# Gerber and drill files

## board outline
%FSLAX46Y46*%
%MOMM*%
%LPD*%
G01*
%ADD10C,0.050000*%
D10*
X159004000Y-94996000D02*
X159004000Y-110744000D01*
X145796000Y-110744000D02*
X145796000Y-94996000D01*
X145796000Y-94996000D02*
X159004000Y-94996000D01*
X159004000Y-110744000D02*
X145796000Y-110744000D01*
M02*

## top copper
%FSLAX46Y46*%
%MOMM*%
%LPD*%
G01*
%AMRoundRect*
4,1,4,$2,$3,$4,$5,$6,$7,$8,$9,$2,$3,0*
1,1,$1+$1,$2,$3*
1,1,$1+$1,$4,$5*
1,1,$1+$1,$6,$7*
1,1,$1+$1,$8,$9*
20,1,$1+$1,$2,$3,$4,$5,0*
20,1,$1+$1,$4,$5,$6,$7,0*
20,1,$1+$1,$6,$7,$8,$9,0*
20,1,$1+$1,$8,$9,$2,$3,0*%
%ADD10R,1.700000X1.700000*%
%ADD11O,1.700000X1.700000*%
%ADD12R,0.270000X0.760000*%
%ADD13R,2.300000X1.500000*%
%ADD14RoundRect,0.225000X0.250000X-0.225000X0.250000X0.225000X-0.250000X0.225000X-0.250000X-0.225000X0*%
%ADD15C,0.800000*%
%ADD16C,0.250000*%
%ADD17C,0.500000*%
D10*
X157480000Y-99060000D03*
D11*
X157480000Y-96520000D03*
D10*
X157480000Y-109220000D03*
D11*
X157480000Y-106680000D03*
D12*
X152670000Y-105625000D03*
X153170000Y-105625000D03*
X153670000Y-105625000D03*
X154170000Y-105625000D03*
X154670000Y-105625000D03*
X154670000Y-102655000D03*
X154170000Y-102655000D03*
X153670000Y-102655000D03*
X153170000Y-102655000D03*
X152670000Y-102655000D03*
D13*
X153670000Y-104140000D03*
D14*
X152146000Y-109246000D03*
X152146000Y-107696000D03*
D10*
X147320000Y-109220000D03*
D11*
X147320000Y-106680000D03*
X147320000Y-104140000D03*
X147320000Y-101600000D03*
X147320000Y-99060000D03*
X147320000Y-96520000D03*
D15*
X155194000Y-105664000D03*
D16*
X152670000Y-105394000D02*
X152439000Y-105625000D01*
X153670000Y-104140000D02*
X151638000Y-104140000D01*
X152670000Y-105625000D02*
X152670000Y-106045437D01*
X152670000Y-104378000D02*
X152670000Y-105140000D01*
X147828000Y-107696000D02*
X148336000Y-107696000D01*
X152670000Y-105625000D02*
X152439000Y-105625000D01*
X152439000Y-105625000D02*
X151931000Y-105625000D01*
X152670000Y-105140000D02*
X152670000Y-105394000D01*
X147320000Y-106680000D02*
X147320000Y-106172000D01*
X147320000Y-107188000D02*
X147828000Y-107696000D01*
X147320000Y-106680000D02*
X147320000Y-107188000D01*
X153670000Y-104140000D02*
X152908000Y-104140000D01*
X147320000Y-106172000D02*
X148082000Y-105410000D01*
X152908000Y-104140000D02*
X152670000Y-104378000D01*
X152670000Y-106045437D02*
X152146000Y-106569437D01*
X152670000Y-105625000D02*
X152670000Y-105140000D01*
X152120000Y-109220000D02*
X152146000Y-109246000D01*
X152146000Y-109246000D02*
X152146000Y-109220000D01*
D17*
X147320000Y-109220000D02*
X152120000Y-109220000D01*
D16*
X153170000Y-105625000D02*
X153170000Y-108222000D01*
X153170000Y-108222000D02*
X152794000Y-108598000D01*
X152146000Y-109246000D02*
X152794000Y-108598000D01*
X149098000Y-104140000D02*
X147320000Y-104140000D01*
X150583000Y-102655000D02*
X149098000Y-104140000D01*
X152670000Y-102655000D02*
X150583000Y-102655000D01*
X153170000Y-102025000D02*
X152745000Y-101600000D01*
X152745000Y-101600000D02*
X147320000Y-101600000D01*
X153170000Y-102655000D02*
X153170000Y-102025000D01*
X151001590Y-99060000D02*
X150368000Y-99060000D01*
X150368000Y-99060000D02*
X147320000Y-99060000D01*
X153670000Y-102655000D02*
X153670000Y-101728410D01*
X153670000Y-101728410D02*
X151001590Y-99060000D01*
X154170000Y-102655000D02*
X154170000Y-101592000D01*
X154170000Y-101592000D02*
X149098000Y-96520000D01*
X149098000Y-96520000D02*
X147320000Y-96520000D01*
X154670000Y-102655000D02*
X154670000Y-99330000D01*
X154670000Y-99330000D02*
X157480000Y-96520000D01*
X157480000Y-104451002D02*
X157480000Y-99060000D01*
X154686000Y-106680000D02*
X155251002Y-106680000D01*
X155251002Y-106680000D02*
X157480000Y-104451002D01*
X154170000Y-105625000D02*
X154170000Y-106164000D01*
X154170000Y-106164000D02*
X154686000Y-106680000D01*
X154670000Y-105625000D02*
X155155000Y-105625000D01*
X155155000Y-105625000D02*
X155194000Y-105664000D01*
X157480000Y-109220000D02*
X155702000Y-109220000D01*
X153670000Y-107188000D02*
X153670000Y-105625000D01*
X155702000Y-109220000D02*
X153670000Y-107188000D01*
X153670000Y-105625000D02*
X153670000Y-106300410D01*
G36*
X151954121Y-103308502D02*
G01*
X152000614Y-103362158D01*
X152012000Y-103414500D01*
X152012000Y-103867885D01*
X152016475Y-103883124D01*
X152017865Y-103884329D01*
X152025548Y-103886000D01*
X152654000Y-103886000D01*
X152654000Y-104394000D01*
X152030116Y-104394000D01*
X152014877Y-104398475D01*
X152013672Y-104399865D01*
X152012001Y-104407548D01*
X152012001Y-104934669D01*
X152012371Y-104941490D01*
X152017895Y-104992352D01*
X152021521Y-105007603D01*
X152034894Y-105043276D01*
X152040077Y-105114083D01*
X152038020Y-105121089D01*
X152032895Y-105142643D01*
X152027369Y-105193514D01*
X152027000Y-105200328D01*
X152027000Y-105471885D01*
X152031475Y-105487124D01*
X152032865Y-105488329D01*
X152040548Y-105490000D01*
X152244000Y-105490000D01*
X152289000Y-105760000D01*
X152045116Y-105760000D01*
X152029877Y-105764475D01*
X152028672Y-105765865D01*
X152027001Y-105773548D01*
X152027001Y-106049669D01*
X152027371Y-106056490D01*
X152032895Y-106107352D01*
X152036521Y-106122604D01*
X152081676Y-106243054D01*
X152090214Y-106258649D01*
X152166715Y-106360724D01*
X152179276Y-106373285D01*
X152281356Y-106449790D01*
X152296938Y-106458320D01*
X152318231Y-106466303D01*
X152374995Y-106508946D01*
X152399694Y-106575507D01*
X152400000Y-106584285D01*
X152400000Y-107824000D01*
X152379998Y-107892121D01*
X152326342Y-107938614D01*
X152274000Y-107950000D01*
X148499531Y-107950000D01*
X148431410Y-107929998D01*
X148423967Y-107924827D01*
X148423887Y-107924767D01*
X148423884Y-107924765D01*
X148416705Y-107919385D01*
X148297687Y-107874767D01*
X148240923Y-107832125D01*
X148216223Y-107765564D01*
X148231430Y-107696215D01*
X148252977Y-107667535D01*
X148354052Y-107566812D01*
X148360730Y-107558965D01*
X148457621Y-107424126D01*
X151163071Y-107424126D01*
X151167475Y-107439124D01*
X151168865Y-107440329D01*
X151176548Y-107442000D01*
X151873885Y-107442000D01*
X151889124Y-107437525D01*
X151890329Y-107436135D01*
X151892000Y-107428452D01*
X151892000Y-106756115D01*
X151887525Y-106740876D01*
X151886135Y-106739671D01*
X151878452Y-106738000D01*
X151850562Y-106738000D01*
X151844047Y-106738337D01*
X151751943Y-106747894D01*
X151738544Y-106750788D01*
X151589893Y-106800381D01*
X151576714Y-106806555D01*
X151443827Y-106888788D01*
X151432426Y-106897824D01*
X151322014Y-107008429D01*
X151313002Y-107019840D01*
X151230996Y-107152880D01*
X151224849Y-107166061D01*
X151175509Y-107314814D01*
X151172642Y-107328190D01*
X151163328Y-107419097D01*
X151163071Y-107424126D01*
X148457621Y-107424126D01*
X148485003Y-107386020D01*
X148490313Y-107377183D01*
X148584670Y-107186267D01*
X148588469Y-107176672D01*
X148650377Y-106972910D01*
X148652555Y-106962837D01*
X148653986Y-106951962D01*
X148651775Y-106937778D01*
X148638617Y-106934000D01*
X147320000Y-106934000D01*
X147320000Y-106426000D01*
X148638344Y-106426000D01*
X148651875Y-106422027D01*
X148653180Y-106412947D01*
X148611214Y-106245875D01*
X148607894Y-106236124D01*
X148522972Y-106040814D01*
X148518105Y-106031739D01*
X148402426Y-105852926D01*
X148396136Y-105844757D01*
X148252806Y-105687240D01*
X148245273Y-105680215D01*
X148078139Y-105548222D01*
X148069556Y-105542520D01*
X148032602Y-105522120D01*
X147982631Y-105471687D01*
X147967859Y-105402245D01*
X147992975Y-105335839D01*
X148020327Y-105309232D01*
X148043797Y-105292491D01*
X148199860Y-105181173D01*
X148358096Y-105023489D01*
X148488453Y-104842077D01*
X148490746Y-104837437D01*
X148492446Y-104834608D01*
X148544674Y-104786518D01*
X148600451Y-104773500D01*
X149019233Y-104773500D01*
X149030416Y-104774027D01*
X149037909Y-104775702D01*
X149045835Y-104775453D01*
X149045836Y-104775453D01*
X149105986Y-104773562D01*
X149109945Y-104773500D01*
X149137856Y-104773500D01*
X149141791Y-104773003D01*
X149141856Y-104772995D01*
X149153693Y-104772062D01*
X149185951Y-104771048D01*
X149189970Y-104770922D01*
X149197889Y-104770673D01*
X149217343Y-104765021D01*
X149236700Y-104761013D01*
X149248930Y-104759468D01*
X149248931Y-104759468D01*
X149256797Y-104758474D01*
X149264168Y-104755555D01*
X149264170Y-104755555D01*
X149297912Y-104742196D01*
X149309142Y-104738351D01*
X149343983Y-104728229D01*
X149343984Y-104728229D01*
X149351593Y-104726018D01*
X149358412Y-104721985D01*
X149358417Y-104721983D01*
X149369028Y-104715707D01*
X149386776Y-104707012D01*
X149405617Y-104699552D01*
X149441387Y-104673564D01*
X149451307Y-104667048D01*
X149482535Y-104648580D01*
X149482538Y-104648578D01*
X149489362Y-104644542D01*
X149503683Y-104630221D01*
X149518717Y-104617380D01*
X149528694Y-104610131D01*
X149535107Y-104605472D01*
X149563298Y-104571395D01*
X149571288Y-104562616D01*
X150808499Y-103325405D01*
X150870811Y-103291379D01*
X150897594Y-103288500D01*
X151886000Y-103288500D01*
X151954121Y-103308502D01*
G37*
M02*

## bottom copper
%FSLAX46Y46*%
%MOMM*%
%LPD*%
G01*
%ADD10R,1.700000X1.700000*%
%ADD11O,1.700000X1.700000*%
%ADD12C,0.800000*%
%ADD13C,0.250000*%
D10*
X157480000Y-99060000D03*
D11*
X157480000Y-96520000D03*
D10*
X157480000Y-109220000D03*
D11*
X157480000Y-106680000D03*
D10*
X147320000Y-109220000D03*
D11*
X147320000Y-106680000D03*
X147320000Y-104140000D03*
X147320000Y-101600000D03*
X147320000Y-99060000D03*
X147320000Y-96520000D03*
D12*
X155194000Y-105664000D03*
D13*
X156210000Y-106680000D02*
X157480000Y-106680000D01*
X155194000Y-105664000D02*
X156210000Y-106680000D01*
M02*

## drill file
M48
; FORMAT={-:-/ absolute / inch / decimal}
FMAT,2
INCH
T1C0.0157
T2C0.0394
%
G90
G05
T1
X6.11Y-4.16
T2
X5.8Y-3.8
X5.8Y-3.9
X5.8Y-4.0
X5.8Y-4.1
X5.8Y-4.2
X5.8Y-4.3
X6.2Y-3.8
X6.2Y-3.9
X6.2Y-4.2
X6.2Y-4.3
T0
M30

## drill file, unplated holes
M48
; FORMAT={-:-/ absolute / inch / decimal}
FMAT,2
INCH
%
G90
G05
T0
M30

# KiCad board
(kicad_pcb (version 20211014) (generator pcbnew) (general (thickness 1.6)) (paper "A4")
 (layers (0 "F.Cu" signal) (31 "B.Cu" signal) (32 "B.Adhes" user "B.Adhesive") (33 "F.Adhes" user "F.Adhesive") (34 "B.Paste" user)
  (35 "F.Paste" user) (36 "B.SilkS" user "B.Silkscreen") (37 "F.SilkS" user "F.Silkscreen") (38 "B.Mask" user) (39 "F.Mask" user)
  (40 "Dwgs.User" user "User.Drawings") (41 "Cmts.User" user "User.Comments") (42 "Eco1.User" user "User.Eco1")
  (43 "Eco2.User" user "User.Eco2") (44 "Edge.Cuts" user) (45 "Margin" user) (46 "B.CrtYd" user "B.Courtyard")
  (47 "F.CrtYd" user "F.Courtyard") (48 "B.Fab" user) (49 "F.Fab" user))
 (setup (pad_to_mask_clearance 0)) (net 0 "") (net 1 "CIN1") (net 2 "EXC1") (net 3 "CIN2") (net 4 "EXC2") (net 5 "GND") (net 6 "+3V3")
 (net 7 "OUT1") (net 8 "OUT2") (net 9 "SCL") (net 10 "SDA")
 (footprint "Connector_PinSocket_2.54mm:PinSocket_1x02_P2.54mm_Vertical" (layer "F.Cu") (at 157.48 99.06 180)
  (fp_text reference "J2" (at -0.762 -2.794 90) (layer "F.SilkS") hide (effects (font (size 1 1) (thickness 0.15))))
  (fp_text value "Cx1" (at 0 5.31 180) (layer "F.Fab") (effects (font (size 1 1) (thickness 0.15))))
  (pad "1" thru_hole rect locked (at 0 0 180) (size 1.7 1.7) (drill 1) (layers *.Cu *.Mask) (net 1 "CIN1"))
  (pad "2" thru_hole oval locked (at 0 2.54 180) (size 1.7 1.7) (drill 1) (layers *.Cu *.Mask) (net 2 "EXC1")))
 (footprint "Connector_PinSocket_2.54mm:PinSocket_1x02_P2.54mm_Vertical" (layer "F.Cu") (at 157.48 109.22 180)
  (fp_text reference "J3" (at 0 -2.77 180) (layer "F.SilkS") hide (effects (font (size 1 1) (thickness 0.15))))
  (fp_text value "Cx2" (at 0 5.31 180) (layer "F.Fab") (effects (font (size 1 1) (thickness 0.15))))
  (pad "1" thru_hole rect locked (at 0 0 180) (size 1.7 1.7) (drill 1) (layers *.Cu *.Mask) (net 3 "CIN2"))
  (pad "2" thru_hole oval locked (at 0 2.54 180) (size 1.7 1.7) (drill 1) (layers *.Cu *.Mask) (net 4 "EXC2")))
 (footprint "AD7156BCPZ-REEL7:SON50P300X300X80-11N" (layer "F.Cu") (at 153.67 104.14 90)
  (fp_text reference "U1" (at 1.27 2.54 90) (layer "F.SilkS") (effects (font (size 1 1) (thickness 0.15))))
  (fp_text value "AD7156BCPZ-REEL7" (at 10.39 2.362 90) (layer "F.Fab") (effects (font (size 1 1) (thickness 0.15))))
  (pad "1" smd rect locked (at -1.485 -1 90) (size 0.76 0.27) (layers "F.Cu" "F.Paste" "F.Mask") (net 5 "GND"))
  (pad "2" smd rect locked (at -1.485 -0.5 90) (size 0.76 0.27) (layers "F.Cu" "F.Paste" "F.Mask") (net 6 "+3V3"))
  (pad "3" smd rect locked (at -1.485 0 90) (size 0.76 0.27) (layers "F.Cu" "F.Paste" "F.Mask") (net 3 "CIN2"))
  (pad "4" smd rect locked (at -1.485 0.5 90) (size 0.76 0.27) (layers "F.Cu" "F.Paste" "F.Mask") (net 1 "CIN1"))
  (pad "5" smd rect locked (at -1.485 1 90) (size 0.76 0.27) (layers "F.Cu" "F.Paste" "F.Mask") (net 4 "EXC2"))
  (pad "6" smd rect locked (at 1.485 1 90) (size 0.76 0.27) (layers "F.Cu" "F.Paste" "F.Mask") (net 2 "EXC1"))
  (pad "7" smd rect locked (at 1.485 0.5 90) (size 0.76 0.27) (layers "F.Cu" "F.Paste" "F.Mask") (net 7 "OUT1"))
  (pad "8" smd rect locked (at 1.485 0 90) (size 0.76 0.27) (layers "F.Cu" "F.Paste" "F.Mask") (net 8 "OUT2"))
  (pad "9" smd rect locked (at 1.485 -0.5 90) (size 0.76 0.27) (layers "F.Cu" "F.Paste" "F.Mask") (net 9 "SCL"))
  (pad "10" smd rect locked (at 1.485 -1 90) (size 0.76 0.27) (layers "F.Cu" "F.Paste" "F.Mask") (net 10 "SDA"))
  (pad "11" smd rect locked (at 0 0 90) (size 1.5 2.3) (layers "F.Cu" "F.Mask") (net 5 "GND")))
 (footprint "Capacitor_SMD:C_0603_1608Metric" (layer "F.Cu") (at 152.146 108.471 90)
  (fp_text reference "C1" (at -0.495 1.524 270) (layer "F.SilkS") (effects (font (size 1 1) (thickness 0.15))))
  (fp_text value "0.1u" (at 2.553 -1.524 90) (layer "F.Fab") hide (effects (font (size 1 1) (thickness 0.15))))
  (pad "1" smd roundrect locked (at -0.775 0 90) (size 0.9 0.95) (layers "F.Cu" "F.Paste" "F.Mask") (roundrect_rratio 0.25) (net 6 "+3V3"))
  (pad "2" smd roundrect locked (at 0.775 0 90) (size 0.9 0.95) (layers "F.Cu" "F.Paste" "F.Mask") (roundrect_rratio 0.25) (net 5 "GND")))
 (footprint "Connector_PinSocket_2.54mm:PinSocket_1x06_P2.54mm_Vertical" (layer "B.Cu") (at 147.32 109.22)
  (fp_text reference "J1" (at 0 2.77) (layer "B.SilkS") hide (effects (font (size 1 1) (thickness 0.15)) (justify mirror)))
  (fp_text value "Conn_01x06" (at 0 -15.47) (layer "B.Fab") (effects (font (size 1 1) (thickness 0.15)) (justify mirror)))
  (pad "1" thru_hole rect locked (at 0 0) (size 1.7 1.7) (drill 1) (layers *.Cu *.Mask) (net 6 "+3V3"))
  (pad "2" thru_hole oval locked (at 0 -2.54) (size 1.7 1.7) (drill 1) (layers *.Cu *.Mask) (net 5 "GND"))
  (pad "3" thru_hole oval locked (at 0 -5.08) (size 1.7 1.7) (drill 1) (layers *.Cu *.Mask) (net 10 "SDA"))
  (pad "4" thru_hole oval locked (at 0 -7.62) (size 1.7 1.7) (drill 1) (layers *.Cu *.Mask) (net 9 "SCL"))
  (pad "5" thru_hole oval locked (at 0 -10.16) (size 1.7 1.7) (drill 1) (layers *.Cu *.Mask) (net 8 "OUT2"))
  (pad "6" thru_hole oval locked (at 0 -12.7) (size 1.7 1.7) (drill 1) (layers *.Cu *.Mask) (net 7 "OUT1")))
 (gr_line (start 159.004 94.996) (end 159.004 110.744) (layer "Edge.Cuts") (width 0.05))
 (gr_line (start 145.796 110.744) (end 145.796 94.996) (layer "Edge.Cuts") (width 0.05))
 (gr_line (start 145.796 94.996) (end 159.004 94.996) (layer "Edge.Cuts") (width 0.05))
 (gr_line (start 159.004 110.744) (end 145.796 110.744) (layer "Edge.Cuts") (width 0.05))
 (segment (start 152.67 105.394) (end 152.439 105.625) (width 0.25) (layer "F.Cu") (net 5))
 (segment (start 153.67 104.14) (end 151.638 104.14) (width 0.25) (layer "F.Cu") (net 5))
 (segment (start 152.67 105.625) (end 152.67 106.045437) (width 0.25) (layer "F.Cu") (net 5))
 (segment (start 152.67 104.378) (end 152.67 105.14) (width 0.25) (layer "F.Cu") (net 5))
 (segment (start 147.828 107.696) (end 148.336 107.696) (width 0.25) (layer "F.Cu") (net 5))
 (segment (start 152.67 105.625) (end 152.439 105.625) (width 0.25) (layer "F.Cu") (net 5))
 (segment (start 152.439 105.625) (end 151.931 105.625) (width 0.25) (layer "F.Cu") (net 5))
 (segment (start 152.67 105.14) (end 152.67 105.394) (width 0.25) (layer "F.Cu") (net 5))
 (segment (start 147.32 106.68) (end 147.32 106.172) (width 0.25) (layer "F.Cu") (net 5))
 (segment (start 147.32 107.188) (end 147.828 107.696) (width 0.25) (layer "F.Cu") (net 5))
 (segment (start 147.32 106.68) (end 147.32 107.188) (width 0.25) (layer "F.Cu") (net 5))
 (segment (start 153.67 104.14) (end 152.908 104.14) (width 0.25) (layer "F.Cu") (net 5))
 (segment (start 147.32 106.172) (end 148.082 105.41) (width 0.25) (layer "F.Cu") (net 5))
 (segment (start 152.908 104.14) (end 152.67 104.378) (width 0.25) (layer "F.Cu") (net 5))
 (segment (start 152.67 106.045437) (end 152.146 106.569437) (width 0.25) (layer "F.Cu") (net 5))
 (segment (start 152.67 105.625) (end 152.67 105.14) (width 0.25) (layer "F.Cu") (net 5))
 (segment (start 152.12 109.22) (end 152.146 109.246) (width 0.25) (layer "F.Cu") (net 6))
 (segment (start 152.146 109.246) (end 152.146 109.22) (width 0.25) (layer "F.Cu") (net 6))
 (segment (start 147.32 109.22) (end 152.12 109.22) (width 0.5) (layer "F.Cu") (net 6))
 (segment (start 153.17 105.625) (end 153.17 108.222) (width 0.25) (layer "F.Cu") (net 6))
 (segment (start 153.17 108.222) (end 152.794 108.598) (width 0.25) (layer "F.Cu") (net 6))
 (segment (start 152.146 109.246) (end 152.794 108.598) (width 0.25) (layer "F.Cu") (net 6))
 (segment (start 149.098 104.14) (end 147.32 104.14) (width 0.25) (layer "F.Cu") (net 10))
 (segment (start 150.583 102.655) (end 149.098 104.14) (width 0.25) (layer "F.Cu") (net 10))
 (segment (start 152.67 102.655) (end 150.583 102.655) (width 0.25) (layer "F.Cu") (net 10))
 (segment (start 153.17 102.025) (end 152.745 101.6) (width 0.25) (layer "F.Cu") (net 9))
 (segment (start 152.745 101.6) (end 147.32 101.6) (width 0.25) (layer "F.Cu") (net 9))
 (segment (start 153.17 102.655) (end 153.17 102.025) (width 0.25) (layer "F.Cu") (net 9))
 (segment (start 151.00159 99.06) (end 150.368 99.06) (width 0.25) (layer "F.Cu") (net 8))
 (segment (start 150.368 99.06) (end 147.32 99.06) (width 0.25) (layer "F.Cu") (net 8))
 (segment (start 153.67 102.655) (end 153.67 101.72841) (width 0.25) (layer "F.Cu") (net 8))
 (segment (start 153.67 101.72841) (end 151.00159 99.06) (width 0.25) (layer "F.Cu") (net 8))
 (segment (start 154.17 102.655) (end 154.17 101.592) (width 0.25) (layer "F.Cu") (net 7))
 (segment (start 154.17 101.592) (end 149.098 96.52) (width 0.25) (layer "F.Cu") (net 7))
 (segment (start 149.098 96.52) (end 147.32 96.52) (width 0.25) (layer "F.Cu") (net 7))
 (segment (start 154.67 102.655) (end 154.67 99.33) (width 0.25) (layer "F.Cu") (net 2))
 (segment (start 154.67 99.33) (end 157.48 96.52) (width 0.25) (layer "F.Cu") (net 2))
 (segment (start 157.48 104.451002) (end 157.48 99.06) (width 0.25) (layer "F.Cu") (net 1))
 (segment (start 154.686 106.68) (end 155.251002 106.68) (width 0.25) (layer "F.Cu") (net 1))
 (segment (start 155.251002 106.68) (end 157.48 104.451002) (width 0.25) (layer "F.Cu") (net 1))
 (segment (start 154.17 105.625) (end 154.17 106.164) (width 0.25) (layer "F.Cu") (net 1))
 (segment (start 154.17 106.164) (end 154.686 106.68) (width 0.25) (layer "F.Cu") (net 1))
 (segment (start 154.67 105.625) (end 155.155 105.625) (width 0.25) (layer "F.Cu") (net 4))
 (segment (start 155.155 105.625) (end 155.194 105.664) (width 0.25) (layer "F.Cu") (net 4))
 (via (at 155.194 105.664) (size 0.8) (drill 0.4) (layers "F.Cu" "B.Cu") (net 4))
 (segment (start 156.21 106.68) (end 157.48 106.68) (width 0.25) (layer "B.Cu") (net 4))
 (segment (start 155.194 105.664) (end 156.21 106.68) (width 0.25) (layer "B.Cu") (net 4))
 (segment (start 157.48 109.22) (end 155.702 109.22) (width 0.25) (layer "F.Cu") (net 3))
 (segment (start 153.67 107.188) (end 153.67 105.625) (width 0.25) (layer "F.Cu") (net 3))
 (segment (start 155.702 109.22) (end 153.67 107.188) (width 0.25) (layer "F.Cu") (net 3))
 (segment (start 153.67 105.625) (end 153.67 106.30041) (width 0.25) (layer "F.Cu") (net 3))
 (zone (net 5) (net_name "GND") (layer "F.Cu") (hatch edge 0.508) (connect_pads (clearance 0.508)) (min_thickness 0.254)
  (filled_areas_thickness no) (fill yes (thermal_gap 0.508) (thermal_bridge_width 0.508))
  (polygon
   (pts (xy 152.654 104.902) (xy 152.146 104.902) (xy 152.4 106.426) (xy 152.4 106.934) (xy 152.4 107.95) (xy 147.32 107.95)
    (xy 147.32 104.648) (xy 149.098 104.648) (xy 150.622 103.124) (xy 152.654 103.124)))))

